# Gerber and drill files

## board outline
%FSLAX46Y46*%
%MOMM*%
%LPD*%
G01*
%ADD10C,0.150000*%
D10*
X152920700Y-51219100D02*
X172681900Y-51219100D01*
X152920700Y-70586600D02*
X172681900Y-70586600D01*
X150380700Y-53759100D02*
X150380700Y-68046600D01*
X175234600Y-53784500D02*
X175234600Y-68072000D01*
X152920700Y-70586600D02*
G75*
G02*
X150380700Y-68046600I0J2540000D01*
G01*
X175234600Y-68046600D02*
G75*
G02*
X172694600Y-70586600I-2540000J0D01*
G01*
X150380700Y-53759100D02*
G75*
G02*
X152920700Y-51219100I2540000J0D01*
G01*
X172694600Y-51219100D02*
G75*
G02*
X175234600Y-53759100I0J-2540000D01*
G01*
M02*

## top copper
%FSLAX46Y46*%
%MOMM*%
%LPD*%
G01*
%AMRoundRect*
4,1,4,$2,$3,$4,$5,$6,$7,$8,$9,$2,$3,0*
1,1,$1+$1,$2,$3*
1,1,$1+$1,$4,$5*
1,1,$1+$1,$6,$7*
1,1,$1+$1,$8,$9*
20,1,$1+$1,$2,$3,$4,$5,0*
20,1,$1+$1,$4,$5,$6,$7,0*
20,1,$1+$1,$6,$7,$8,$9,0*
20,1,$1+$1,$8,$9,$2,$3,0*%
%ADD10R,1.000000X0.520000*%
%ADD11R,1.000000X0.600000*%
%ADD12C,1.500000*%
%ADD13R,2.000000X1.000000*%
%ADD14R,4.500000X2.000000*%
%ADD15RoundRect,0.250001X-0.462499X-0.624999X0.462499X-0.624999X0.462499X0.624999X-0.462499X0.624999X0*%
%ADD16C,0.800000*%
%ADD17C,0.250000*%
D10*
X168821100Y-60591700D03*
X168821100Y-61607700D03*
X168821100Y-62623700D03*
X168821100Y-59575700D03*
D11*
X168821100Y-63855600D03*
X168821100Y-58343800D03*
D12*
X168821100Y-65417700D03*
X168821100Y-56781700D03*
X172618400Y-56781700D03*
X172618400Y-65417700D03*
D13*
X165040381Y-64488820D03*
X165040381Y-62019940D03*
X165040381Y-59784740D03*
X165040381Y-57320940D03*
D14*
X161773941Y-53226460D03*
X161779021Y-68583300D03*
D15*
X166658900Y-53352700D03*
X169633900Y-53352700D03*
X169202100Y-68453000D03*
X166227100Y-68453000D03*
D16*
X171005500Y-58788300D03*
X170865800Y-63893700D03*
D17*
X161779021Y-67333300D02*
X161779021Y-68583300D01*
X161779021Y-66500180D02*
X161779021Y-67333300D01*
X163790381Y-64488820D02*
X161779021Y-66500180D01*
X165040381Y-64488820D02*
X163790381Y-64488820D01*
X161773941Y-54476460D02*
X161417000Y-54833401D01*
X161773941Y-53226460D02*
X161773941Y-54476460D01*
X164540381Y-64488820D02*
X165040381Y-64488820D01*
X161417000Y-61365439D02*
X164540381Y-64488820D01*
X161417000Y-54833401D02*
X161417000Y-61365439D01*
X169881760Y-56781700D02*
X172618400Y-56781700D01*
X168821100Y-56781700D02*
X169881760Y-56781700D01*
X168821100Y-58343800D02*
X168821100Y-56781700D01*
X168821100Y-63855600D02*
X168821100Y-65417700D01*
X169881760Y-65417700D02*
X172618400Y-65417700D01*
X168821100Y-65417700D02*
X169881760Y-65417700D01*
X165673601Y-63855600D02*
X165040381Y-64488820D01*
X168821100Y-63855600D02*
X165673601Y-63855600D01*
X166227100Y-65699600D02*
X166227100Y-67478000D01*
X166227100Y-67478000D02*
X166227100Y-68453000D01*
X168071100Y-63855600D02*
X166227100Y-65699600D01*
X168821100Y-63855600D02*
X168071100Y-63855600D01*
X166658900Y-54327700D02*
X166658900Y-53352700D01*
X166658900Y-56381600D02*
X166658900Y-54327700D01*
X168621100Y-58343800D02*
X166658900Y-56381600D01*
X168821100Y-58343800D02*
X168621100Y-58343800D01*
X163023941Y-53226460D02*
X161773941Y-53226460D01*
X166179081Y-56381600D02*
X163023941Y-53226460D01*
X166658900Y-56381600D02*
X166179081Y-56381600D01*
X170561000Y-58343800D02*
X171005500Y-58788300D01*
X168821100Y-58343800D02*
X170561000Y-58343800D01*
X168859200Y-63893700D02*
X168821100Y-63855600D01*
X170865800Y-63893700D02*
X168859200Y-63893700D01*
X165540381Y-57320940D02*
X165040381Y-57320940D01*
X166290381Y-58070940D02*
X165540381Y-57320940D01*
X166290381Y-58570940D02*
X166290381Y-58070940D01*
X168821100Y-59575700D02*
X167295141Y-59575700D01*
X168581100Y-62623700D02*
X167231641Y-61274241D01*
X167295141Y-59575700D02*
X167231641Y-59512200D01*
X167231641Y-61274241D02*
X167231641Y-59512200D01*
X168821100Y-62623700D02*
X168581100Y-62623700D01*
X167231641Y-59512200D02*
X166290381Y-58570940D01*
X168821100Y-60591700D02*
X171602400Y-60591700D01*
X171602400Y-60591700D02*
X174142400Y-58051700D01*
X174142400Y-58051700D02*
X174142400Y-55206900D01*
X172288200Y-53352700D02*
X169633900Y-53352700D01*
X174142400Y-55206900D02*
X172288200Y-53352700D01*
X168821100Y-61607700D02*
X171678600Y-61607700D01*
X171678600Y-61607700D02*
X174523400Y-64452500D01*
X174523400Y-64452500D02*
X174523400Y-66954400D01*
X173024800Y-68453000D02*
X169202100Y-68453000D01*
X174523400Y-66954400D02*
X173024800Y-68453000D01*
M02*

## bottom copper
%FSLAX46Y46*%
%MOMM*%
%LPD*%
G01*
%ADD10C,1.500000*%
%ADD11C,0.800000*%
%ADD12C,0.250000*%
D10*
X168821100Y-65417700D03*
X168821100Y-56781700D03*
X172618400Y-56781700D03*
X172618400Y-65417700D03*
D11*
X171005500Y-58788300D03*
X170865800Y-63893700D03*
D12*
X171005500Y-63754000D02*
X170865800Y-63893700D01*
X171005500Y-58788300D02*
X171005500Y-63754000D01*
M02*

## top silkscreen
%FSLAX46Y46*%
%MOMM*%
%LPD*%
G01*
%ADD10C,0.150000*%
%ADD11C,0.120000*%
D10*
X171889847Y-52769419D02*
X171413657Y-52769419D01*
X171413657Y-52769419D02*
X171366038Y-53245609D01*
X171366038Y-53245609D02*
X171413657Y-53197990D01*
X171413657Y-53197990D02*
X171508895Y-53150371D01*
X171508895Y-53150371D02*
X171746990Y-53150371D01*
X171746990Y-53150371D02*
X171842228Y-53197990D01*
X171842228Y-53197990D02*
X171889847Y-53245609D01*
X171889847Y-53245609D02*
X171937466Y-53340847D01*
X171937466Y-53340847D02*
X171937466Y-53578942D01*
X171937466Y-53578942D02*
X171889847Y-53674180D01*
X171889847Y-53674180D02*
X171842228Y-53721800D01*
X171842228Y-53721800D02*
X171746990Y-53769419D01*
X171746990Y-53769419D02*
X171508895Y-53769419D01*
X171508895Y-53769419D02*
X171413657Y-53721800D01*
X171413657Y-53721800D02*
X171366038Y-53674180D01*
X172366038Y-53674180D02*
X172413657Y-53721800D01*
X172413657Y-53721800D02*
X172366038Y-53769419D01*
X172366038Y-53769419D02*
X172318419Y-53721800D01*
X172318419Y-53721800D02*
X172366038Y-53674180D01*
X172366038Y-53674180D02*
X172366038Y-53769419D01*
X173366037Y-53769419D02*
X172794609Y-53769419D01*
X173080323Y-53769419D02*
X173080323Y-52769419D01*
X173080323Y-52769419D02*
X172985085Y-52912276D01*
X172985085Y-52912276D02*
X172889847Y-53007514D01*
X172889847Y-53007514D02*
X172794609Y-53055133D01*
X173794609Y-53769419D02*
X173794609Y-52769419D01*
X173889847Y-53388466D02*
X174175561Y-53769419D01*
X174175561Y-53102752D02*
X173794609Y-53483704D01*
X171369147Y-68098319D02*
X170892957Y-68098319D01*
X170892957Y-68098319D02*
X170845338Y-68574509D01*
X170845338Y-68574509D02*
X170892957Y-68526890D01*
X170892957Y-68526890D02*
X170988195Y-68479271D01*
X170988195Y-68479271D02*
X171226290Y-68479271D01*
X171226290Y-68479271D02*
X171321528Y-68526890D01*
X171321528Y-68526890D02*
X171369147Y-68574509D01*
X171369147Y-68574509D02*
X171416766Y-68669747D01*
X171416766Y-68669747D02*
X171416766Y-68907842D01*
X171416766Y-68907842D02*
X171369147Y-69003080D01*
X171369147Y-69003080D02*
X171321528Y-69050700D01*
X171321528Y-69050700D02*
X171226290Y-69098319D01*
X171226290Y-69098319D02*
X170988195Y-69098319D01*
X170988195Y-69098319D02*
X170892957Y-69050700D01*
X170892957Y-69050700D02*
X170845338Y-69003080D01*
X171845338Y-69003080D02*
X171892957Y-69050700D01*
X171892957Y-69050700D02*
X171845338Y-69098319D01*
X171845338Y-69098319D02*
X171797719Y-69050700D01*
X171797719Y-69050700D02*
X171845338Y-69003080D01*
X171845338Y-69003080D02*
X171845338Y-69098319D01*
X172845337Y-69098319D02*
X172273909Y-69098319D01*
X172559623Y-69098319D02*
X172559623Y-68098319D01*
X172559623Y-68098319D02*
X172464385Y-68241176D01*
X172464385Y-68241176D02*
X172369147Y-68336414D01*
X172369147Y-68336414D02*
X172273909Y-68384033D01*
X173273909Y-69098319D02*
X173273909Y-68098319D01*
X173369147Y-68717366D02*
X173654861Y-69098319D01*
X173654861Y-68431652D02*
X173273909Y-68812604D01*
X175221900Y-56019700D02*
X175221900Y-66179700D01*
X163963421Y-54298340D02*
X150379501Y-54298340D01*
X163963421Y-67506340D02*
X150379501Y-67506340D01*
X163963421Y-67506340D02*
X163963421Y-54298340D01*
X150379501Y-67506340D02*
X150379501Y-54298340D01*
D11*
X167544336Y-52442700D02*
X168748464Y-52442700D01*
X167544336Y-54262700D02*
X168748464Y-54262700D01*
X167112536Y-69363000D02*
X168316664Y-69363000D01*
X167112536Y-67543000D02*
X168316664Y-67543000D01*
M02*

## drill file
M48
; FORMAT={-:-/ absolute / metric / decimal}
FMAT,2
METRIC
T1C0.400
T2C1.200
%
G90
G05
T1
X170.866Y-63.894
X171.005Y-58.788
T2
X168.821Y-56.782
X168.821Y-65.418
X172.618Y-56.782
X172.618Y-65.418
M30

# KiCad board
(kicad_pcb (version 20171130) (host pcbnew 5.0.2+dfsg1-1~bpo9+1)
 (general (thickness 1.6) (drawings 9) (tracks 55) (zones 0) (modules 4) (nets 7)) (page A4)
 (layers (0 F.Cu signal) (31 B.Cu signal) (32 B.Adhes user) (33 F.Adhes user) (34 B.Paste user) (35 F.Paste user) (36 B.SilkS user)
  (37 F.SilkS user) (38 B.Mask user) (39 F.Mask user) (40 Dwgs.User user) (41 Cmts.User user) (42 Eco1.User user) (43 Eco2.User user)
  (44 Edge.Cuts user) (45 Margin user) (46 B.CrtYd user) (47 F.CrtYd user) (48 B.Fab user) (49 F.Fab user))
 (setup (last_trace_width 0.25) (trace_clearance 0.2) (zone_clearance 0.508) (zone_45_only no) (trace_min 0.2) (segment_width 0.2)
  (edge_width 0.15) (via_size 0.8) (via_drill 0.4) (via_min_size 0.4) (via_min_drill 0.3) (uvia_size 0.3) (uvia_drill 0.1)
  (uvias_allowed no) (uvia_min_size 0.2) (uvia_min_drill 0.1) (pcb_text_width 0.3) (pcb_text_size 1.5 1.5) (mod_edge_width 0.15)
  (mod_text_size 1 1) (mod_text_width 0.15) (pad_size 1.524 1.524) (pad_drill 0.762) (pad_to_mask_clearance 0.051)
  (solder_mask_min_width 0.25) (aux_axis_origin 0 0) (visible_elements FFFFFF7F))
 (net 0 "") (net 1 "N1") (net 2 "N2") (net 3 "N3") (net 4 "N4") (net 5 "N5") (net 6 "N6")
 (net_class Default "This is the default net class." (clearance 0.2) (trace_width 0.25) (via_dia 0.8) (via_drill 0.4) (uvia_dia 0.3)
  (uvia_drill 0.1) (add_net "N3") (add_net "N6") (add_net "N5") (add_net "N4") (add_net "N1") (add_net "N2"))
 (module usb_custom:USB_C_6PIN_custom (layer F.Cu) (at 168.8211 61.0997 270)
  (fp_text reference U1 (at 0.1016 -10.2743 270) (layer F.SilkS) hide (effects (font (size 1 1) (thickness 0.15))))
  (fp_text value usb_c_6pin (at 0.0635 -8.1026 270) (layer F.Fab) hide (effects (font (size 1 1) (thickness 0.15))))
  (fp_line (start -5.08 -6.4008) (end 5.08 -6.4008) (layer F.SilkS) (width 0.15))
  (pad 3 smd rect (at -0.508 0 270) (size 0.52 1) (layers F.Cu F.Paste F.Mask) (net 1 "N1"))
  (pad 4 smd rect (at 0.508 0 270) (size 0.52 1) (layers F.Cu F.Paste F.Mask) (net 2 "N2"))
  (pad 2 smd rect (at 1.524 0 270) (size 0.52 1) (layers F.Cu F.Paste F.Mask) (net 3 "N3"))
  (pad 2 smd rect (at -1.524 0 270) (size 0.52 1) (layers F.Cu F.Paste F.Mask) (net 3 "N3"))
  (pad 1 smd rect (at 2.7559 0 270) (size 0.6 1) (layers F.Cu F.Paste F.Mask) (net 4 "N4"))
  (pad 1 smd rect (at -2.7559 0 270) (size 0.6 1) (layers F.Cu F.Paste F.Mask) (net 4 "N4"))
  (pad 1 thru_hole circle (at 4.318 0 270) (size 1.5 1.5) (drill 1.2) (layers *.Cu *.Mask) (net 4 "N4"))
  (pad 1 thru_hole circle (at -4.318 0 270) (size 1.5 1.5) (drill 1.2) (layers *.Cu *.Mask) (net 4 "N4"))
  (pad 1 thru_hole circle (at -4.318 -3.7973 270) (size 1.5 1.5) (drill 1.2) (layers *.Cu *.Mask) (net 4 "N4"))
  (pad 1 thru_hole circle (at 4.318 -3.7973 270) (size 1.5 1.5) (drill 1.2) (layers *.Cu *.Mask) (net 4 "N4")))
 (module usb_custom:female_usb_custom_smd (layer F.Cu) (at 163.079501 60.90234 90)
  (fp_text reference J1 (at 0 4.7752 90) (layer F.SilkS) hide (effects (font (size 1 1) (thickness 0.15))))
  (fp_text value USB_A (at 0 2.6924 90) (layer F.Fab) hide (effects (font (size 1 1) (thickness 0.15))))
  (fp_line (start 6.604 0.88392) (end 6.604 -12.7) (layer F.SilkS) (width 0.15))
  (fp_line (start -6.604 0.88392) (end -6.604 -12.7) (layer F.SilkS) (width 0.15))
  (fp_line (start -6.604 0.88392) (end 6.604 0.88392) (layer F.SilkS) (width 0.15))
  (fp_line (start -6.604 -12.7) (end 6.604 -12.7) (layer F.SilkS) (width 0.15))
  (pad 4 smd rect (at -3.58648 1.96088 90) (size 1 2) (layers F.Cu F.Paste F.Mask) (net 4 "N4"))
  (pad 3 smd rect (at -1.1176 1.96088 90) (size 1 2) (layers F.Cu F.Paste F.Mask) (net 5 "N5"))
  (pad 2 smd rect (at 1.1176 1.96088 90) (size 1 2) (layers F.Cu F.Paste F.Mask) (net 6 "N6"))
  (pad 1 smd rect (at 3.5814 1.96088 90) (size 1 2) (layers F.Cu F.Paste F.Mask) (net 3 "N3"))
  (pad 5 smd rect (at 7.67588 -1.30556 90) (size 2 4.5) (layers F.Cu F.Paste F.Mask) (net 4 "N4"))
  (pad 5 smd rect (at -7.68096 -1.30048 90) (size 2 4.5) (layers F.Cu F.Paste F.Mask) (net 4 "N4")))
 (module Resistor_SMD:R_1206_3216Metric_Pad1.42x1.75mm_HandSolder (layer F.Cu) (at 168.1464 53.3527)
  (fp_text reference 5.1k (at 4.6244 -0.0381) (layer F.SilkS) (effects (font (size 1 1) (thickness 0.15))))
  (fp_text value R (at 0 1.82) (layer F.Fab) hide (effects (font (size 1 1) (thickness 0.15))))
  (fp_line (start -0.602064 -0.91) (end 0.602064 -0.91) (layer F.SilkS) (width 0.12))
  (fp_line (start -0.602064 0.91) (end 0.602064 0.91) (layer F.SilkS) (width 0.12))
  (pad 1 smd roundrect (at -1.4875 0) (size 1.425 1.75) (layers F.Cu F.Paste F.Mask) (roundrect_rratio 0.175439) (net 4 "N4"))
  (pad 2 smd roundrect (at 1.4875 0) (size 1.425 1.75) (layers F.Cu F.Paste F.Mask) (roundrect_rratio 0.175439) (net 1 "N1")))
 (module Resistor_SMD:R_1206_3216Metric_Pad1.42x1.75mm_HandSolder (layer F.Cu) (at 167.7146 68.453)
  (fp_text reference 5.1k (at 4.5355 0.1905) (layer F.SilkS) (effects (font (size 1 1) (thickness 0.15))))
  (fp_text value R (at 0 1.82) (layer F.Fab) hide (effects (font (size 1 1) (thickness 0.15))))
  (fp_line (start -0.602064 0.91) (end 0.602064 0.91) (layer F.SilkS) (width 0.12))
  (fp_line (start -0.602064 -0.91) (end 0.602064 -0.91) (layer F.SilkS) (width 0.12))
  (pad 2 smd roundrect (at 1.4875 0) (size 1.425 1.75) (layers F.Cu F.Paste F.Mask) (roundrect_rratio 0.175439) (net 2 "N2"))
  (pad 1 smd roundrect (at -1.4875 0) (size 1.425 1.75) (layers F.Cu F.Paste F.Mask) (roundrect_rratio 0.175439) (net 4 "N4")))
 (gr_line (start 152.9207 51.2191) (end 172.6819 51.2191) (layer Edge.Cuts) (width 0.15))
 (gr_line (start 152.9207 70.5866) (end 172.6819 70.5866) (layer Edge.Cuts) (width 0.15))
 (gr_line (start 150.3807 53.7591) (end 150.3807 68.0466) (layer Edge.Cuts) (width 0.15))
 (gr_line (start 175.2346 53.7845) (end 175.2346 68.072) (layer Edge.Cuts) (width 0.15))
 (gr_arc (start 152.9207 68.0466) (end 150.3807 68.0466) (angle -90) (layer Edge.Cuts) (width 0.15))
 (gr_arc (start 172.6946 68.0466) (end 172.6946 70.5866) (angle -90) (layer Edge.Cuts) (width 0.15))
 (gr_arc (start 152.9207 53.7591) (end 152.9207 51.2191) (angle -90) (layer Edge.Cuts) (width 0.15))
 (gr_arc (start 172.6946 53.7591) (end 175.2346 53.7591) (angle -90) (layer Edge.Cuts) (width 0.15))
 (segment (start 161.779021 67.3333) (end 161.779021 68.5833) (width 0.25) (layer F.Cu) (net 4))
 (segment (start 161.779021 66.50018) (end 161.779021 67.3333) (width 0.25) (layer F.Cu) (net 4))
 (segment (start 163.790381 64.48882) (end 161.779021 66.50018) (width 0.25) (layer F.Cu) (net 4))
 (segment (start 165.040381 64.48882) (end 163.790381 64.48882) (width 0.25) (layer F.Cu) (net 4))
 (segment (start 161.773941 54.47646) (end 161.417 54.833401) (width 0.25) (layer F.Cu) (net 4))
 (segment (start 161.773941 53.22646) (end 161.773941 54.47646) (width 0.25) (layer F.Cu) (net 4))
 (segment (start 164.540381 64.48882) (end 165.040381 64.48882) (width 0.25) (layer F.Cu) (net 4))
 (segment (start 161.417 61.365439) (end 164.540381 64.48882) (width 0.25) (layer F.Cu) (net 4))
 (segment (start 161.417 54.833401) (end 161.417 61.365439) (width 0.25) (layer F.Cu) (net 4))
 (segment (start 169.88176 56.7817) (end 172.6184 56.7817) (width 0.25) (layer F.Cu) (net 4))
 (segment (start 168.8211 56.7817) (end 169.88176 56.7817) (width 0.25) (layer F.Cu) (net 4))
 (segment (start 168.8211 58.3438) (end 168.8211 56.7817) (width 0.25) (layer F.Cu) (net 4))
 (segment (start 168.8211 63.8556) (end 168.8211 65.4177) (width 0.25) (layer F.Cu) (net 4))
 (segment (start 169.88176 65.4177) (end 172.6184 65.4177) (width 0.25) (layer F.Cu) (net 4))
 (segment (start 168.8211 65.4177) (end 169.88176 65.4177) (width 0.25) (layer F.Cu) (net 4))
 (segment (start 165.673601 63.8556) (end 165.040381 64.48882) (width 0.25) (layer F.Cu) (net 4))
 (segment (start 168.8211 63.8556) (end 165.673601 63.8556) (width 0.25) (layer F.Cu) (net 4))
 (segment (start 166.2271 65.6996) (end 166.2271 67.478) (width 0.25) (layer F.Cu) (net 4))
 (segment (start 166.2271 67.478) (end 166.2271 68.453) (width 0.25) (layer F.Cu) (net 4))
 (segment (start 168.0711 63.8556) (end 166.2271 65.6996) (width 0.25) (layer F.Cu) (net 4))
 (segment (start 168.8211 63.8556) (end 168.0711 63.8556) (width 0.25) (layer F.Cu) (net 4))
 (segment (start 166.6589 54.3277) (end 166.6589 53.3527) (width 0.25) (layer F.Cu) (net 4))
 (segment (start 166.6589 56.3816) (end 166.6589 54.3277) (width 0.25) (layer F.Cu) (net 4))
 (segment (start 168.6211 58.3438) (end 166.6589 56.3816) (width 0.25) (layer F.Cu) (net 4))
 (segment (start 168.8211 58.3438) (end 168.6211 58.3438) (width 0.25) (layer F.Cu) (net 4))
 (segment (start 163.023941 53.22646) (end 161.773941 53.22646) (width 0.25) (layer F.Cu) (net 4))
 (segment (start 166.179081 56.3816) (end 163.023941 53.22646) (width 0.25) (layer F.Cu) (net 4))
 (segment (start 166.6589 56.3816) (end 166.179081 56.3816) (width 0.25) (layer F.Cu) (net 4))
 (via (at 171.0055 58.7883) (size 0.8) (drill 0.4) (layers F.Cu B.Cu) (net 4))
 (segment (start 170.561 58.3438) (end 171.0055 58.7883) (width 0.25) (layer F.Cu) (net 4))
 (segment (start 168.8211 58.3438) (end 170.561 58.3438) (width 0.25) (layer F.Cu) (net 4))
 (via (at 170.8658 63.8937) (size 0.8) (drill 0.4) (layers F.Cu B.Cu) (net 4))
 (segment (start 171.0055 63.754) (end 170.8658 63.8937) (width 0.25) (layer B.Cu) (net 4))
 (segment (start 171.0055 58.7883) (end 171.0055 63.754) (width 0.25) (layer B.Cu) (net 4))
 (segment (start 168.8592 63.8937) (end 168.8211 63.8556) (width 0.25) (layer F.Cu) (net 4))
 (segment (start 170.8658 63.8937) (end 168.8592 63.8937) (width 0.25) (layer F.Cu) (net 4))
 (segment (start 165.540381 57.32094) (end 165.040381 57.32094) (width 0.25) (layer F.Cu) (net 3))
 (segment (start 166.290381 58.07094) (end 165.540381 57.32094) (width 0.25) (layer F.Cu) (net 3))
 (segment (start 166.290381 58.57094) (end 166.290381 58.07094) (width 0.25) (layer F.Cu) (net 3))
 (segment (start 168.8211 59.5757) (end 167.295141 59.5757) (width 0.25) (layer F.Cu) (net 3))
 (segment (start 168.5811 62.6237) (end 167.231641 61.274241) (width 0.25) (layer F.Cu) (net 3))
 (segment (start 167.295141 59.5757) (end 167.231641 59.5122) (width 0.25) (layer F.Cu) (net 3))
 (segment (start 167.231641 61.274241) (end 167.231641 59.5122) (width 0.25) (layer F.Cu) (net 3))
 (segment (start 168.8211 62.6237) (end 168.5811 62.6237) (width 0.25) (layer F.Cu) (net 3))
 (segment (start 167.231641 59.5122) (end 166.290381 58.57094) (width 0.25) (layer F.Cu) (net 3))
 (segment (start 168.8211 60.5917) (end 171.6024 60.5917) (width 0.25) (layer F.Cu) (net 1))
 (segment (start 171.6024 60.5917) (end 174.1424 58.0517) (width 0.25) (layer F.Cu) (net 1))
 (segment (start 174.1424 58.0517) (end 174.1424 55.2069) (width 0.25) (layer F.Cu) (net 1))
 (segment (start 172.2882 53.3527) (end 169.6339 53.3527) (width 0.25) (layer F.Cu) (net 1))
 (segment (start 174.1424 55.2069) (end 172.2882 53.3527) (width 0.25) (layer F.Cu) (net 1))
 (segment (start 168.8211 61.6077) (end 171.6786 61.6077) (width 0.25) (layer F.Cu) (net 2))
 (segment (start 171.6786 61.6077) (end 174.5234 64.4525) (width 0.25) (layer F.Cu) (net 2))
 (segment (start 174.5234 64.4525) (end 174.5234 66.9544) (width 0.25) (layer F.Cu) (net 2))
 (segment (start 173.0248 68.453) (end 169.2021 68.453) (width 0.25) (layer F.Cu) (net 2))
 (segment (start 174.5234 66.9544) (end 173.0248 68.453) (width 0.25) (layer F.Cu) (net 2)))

